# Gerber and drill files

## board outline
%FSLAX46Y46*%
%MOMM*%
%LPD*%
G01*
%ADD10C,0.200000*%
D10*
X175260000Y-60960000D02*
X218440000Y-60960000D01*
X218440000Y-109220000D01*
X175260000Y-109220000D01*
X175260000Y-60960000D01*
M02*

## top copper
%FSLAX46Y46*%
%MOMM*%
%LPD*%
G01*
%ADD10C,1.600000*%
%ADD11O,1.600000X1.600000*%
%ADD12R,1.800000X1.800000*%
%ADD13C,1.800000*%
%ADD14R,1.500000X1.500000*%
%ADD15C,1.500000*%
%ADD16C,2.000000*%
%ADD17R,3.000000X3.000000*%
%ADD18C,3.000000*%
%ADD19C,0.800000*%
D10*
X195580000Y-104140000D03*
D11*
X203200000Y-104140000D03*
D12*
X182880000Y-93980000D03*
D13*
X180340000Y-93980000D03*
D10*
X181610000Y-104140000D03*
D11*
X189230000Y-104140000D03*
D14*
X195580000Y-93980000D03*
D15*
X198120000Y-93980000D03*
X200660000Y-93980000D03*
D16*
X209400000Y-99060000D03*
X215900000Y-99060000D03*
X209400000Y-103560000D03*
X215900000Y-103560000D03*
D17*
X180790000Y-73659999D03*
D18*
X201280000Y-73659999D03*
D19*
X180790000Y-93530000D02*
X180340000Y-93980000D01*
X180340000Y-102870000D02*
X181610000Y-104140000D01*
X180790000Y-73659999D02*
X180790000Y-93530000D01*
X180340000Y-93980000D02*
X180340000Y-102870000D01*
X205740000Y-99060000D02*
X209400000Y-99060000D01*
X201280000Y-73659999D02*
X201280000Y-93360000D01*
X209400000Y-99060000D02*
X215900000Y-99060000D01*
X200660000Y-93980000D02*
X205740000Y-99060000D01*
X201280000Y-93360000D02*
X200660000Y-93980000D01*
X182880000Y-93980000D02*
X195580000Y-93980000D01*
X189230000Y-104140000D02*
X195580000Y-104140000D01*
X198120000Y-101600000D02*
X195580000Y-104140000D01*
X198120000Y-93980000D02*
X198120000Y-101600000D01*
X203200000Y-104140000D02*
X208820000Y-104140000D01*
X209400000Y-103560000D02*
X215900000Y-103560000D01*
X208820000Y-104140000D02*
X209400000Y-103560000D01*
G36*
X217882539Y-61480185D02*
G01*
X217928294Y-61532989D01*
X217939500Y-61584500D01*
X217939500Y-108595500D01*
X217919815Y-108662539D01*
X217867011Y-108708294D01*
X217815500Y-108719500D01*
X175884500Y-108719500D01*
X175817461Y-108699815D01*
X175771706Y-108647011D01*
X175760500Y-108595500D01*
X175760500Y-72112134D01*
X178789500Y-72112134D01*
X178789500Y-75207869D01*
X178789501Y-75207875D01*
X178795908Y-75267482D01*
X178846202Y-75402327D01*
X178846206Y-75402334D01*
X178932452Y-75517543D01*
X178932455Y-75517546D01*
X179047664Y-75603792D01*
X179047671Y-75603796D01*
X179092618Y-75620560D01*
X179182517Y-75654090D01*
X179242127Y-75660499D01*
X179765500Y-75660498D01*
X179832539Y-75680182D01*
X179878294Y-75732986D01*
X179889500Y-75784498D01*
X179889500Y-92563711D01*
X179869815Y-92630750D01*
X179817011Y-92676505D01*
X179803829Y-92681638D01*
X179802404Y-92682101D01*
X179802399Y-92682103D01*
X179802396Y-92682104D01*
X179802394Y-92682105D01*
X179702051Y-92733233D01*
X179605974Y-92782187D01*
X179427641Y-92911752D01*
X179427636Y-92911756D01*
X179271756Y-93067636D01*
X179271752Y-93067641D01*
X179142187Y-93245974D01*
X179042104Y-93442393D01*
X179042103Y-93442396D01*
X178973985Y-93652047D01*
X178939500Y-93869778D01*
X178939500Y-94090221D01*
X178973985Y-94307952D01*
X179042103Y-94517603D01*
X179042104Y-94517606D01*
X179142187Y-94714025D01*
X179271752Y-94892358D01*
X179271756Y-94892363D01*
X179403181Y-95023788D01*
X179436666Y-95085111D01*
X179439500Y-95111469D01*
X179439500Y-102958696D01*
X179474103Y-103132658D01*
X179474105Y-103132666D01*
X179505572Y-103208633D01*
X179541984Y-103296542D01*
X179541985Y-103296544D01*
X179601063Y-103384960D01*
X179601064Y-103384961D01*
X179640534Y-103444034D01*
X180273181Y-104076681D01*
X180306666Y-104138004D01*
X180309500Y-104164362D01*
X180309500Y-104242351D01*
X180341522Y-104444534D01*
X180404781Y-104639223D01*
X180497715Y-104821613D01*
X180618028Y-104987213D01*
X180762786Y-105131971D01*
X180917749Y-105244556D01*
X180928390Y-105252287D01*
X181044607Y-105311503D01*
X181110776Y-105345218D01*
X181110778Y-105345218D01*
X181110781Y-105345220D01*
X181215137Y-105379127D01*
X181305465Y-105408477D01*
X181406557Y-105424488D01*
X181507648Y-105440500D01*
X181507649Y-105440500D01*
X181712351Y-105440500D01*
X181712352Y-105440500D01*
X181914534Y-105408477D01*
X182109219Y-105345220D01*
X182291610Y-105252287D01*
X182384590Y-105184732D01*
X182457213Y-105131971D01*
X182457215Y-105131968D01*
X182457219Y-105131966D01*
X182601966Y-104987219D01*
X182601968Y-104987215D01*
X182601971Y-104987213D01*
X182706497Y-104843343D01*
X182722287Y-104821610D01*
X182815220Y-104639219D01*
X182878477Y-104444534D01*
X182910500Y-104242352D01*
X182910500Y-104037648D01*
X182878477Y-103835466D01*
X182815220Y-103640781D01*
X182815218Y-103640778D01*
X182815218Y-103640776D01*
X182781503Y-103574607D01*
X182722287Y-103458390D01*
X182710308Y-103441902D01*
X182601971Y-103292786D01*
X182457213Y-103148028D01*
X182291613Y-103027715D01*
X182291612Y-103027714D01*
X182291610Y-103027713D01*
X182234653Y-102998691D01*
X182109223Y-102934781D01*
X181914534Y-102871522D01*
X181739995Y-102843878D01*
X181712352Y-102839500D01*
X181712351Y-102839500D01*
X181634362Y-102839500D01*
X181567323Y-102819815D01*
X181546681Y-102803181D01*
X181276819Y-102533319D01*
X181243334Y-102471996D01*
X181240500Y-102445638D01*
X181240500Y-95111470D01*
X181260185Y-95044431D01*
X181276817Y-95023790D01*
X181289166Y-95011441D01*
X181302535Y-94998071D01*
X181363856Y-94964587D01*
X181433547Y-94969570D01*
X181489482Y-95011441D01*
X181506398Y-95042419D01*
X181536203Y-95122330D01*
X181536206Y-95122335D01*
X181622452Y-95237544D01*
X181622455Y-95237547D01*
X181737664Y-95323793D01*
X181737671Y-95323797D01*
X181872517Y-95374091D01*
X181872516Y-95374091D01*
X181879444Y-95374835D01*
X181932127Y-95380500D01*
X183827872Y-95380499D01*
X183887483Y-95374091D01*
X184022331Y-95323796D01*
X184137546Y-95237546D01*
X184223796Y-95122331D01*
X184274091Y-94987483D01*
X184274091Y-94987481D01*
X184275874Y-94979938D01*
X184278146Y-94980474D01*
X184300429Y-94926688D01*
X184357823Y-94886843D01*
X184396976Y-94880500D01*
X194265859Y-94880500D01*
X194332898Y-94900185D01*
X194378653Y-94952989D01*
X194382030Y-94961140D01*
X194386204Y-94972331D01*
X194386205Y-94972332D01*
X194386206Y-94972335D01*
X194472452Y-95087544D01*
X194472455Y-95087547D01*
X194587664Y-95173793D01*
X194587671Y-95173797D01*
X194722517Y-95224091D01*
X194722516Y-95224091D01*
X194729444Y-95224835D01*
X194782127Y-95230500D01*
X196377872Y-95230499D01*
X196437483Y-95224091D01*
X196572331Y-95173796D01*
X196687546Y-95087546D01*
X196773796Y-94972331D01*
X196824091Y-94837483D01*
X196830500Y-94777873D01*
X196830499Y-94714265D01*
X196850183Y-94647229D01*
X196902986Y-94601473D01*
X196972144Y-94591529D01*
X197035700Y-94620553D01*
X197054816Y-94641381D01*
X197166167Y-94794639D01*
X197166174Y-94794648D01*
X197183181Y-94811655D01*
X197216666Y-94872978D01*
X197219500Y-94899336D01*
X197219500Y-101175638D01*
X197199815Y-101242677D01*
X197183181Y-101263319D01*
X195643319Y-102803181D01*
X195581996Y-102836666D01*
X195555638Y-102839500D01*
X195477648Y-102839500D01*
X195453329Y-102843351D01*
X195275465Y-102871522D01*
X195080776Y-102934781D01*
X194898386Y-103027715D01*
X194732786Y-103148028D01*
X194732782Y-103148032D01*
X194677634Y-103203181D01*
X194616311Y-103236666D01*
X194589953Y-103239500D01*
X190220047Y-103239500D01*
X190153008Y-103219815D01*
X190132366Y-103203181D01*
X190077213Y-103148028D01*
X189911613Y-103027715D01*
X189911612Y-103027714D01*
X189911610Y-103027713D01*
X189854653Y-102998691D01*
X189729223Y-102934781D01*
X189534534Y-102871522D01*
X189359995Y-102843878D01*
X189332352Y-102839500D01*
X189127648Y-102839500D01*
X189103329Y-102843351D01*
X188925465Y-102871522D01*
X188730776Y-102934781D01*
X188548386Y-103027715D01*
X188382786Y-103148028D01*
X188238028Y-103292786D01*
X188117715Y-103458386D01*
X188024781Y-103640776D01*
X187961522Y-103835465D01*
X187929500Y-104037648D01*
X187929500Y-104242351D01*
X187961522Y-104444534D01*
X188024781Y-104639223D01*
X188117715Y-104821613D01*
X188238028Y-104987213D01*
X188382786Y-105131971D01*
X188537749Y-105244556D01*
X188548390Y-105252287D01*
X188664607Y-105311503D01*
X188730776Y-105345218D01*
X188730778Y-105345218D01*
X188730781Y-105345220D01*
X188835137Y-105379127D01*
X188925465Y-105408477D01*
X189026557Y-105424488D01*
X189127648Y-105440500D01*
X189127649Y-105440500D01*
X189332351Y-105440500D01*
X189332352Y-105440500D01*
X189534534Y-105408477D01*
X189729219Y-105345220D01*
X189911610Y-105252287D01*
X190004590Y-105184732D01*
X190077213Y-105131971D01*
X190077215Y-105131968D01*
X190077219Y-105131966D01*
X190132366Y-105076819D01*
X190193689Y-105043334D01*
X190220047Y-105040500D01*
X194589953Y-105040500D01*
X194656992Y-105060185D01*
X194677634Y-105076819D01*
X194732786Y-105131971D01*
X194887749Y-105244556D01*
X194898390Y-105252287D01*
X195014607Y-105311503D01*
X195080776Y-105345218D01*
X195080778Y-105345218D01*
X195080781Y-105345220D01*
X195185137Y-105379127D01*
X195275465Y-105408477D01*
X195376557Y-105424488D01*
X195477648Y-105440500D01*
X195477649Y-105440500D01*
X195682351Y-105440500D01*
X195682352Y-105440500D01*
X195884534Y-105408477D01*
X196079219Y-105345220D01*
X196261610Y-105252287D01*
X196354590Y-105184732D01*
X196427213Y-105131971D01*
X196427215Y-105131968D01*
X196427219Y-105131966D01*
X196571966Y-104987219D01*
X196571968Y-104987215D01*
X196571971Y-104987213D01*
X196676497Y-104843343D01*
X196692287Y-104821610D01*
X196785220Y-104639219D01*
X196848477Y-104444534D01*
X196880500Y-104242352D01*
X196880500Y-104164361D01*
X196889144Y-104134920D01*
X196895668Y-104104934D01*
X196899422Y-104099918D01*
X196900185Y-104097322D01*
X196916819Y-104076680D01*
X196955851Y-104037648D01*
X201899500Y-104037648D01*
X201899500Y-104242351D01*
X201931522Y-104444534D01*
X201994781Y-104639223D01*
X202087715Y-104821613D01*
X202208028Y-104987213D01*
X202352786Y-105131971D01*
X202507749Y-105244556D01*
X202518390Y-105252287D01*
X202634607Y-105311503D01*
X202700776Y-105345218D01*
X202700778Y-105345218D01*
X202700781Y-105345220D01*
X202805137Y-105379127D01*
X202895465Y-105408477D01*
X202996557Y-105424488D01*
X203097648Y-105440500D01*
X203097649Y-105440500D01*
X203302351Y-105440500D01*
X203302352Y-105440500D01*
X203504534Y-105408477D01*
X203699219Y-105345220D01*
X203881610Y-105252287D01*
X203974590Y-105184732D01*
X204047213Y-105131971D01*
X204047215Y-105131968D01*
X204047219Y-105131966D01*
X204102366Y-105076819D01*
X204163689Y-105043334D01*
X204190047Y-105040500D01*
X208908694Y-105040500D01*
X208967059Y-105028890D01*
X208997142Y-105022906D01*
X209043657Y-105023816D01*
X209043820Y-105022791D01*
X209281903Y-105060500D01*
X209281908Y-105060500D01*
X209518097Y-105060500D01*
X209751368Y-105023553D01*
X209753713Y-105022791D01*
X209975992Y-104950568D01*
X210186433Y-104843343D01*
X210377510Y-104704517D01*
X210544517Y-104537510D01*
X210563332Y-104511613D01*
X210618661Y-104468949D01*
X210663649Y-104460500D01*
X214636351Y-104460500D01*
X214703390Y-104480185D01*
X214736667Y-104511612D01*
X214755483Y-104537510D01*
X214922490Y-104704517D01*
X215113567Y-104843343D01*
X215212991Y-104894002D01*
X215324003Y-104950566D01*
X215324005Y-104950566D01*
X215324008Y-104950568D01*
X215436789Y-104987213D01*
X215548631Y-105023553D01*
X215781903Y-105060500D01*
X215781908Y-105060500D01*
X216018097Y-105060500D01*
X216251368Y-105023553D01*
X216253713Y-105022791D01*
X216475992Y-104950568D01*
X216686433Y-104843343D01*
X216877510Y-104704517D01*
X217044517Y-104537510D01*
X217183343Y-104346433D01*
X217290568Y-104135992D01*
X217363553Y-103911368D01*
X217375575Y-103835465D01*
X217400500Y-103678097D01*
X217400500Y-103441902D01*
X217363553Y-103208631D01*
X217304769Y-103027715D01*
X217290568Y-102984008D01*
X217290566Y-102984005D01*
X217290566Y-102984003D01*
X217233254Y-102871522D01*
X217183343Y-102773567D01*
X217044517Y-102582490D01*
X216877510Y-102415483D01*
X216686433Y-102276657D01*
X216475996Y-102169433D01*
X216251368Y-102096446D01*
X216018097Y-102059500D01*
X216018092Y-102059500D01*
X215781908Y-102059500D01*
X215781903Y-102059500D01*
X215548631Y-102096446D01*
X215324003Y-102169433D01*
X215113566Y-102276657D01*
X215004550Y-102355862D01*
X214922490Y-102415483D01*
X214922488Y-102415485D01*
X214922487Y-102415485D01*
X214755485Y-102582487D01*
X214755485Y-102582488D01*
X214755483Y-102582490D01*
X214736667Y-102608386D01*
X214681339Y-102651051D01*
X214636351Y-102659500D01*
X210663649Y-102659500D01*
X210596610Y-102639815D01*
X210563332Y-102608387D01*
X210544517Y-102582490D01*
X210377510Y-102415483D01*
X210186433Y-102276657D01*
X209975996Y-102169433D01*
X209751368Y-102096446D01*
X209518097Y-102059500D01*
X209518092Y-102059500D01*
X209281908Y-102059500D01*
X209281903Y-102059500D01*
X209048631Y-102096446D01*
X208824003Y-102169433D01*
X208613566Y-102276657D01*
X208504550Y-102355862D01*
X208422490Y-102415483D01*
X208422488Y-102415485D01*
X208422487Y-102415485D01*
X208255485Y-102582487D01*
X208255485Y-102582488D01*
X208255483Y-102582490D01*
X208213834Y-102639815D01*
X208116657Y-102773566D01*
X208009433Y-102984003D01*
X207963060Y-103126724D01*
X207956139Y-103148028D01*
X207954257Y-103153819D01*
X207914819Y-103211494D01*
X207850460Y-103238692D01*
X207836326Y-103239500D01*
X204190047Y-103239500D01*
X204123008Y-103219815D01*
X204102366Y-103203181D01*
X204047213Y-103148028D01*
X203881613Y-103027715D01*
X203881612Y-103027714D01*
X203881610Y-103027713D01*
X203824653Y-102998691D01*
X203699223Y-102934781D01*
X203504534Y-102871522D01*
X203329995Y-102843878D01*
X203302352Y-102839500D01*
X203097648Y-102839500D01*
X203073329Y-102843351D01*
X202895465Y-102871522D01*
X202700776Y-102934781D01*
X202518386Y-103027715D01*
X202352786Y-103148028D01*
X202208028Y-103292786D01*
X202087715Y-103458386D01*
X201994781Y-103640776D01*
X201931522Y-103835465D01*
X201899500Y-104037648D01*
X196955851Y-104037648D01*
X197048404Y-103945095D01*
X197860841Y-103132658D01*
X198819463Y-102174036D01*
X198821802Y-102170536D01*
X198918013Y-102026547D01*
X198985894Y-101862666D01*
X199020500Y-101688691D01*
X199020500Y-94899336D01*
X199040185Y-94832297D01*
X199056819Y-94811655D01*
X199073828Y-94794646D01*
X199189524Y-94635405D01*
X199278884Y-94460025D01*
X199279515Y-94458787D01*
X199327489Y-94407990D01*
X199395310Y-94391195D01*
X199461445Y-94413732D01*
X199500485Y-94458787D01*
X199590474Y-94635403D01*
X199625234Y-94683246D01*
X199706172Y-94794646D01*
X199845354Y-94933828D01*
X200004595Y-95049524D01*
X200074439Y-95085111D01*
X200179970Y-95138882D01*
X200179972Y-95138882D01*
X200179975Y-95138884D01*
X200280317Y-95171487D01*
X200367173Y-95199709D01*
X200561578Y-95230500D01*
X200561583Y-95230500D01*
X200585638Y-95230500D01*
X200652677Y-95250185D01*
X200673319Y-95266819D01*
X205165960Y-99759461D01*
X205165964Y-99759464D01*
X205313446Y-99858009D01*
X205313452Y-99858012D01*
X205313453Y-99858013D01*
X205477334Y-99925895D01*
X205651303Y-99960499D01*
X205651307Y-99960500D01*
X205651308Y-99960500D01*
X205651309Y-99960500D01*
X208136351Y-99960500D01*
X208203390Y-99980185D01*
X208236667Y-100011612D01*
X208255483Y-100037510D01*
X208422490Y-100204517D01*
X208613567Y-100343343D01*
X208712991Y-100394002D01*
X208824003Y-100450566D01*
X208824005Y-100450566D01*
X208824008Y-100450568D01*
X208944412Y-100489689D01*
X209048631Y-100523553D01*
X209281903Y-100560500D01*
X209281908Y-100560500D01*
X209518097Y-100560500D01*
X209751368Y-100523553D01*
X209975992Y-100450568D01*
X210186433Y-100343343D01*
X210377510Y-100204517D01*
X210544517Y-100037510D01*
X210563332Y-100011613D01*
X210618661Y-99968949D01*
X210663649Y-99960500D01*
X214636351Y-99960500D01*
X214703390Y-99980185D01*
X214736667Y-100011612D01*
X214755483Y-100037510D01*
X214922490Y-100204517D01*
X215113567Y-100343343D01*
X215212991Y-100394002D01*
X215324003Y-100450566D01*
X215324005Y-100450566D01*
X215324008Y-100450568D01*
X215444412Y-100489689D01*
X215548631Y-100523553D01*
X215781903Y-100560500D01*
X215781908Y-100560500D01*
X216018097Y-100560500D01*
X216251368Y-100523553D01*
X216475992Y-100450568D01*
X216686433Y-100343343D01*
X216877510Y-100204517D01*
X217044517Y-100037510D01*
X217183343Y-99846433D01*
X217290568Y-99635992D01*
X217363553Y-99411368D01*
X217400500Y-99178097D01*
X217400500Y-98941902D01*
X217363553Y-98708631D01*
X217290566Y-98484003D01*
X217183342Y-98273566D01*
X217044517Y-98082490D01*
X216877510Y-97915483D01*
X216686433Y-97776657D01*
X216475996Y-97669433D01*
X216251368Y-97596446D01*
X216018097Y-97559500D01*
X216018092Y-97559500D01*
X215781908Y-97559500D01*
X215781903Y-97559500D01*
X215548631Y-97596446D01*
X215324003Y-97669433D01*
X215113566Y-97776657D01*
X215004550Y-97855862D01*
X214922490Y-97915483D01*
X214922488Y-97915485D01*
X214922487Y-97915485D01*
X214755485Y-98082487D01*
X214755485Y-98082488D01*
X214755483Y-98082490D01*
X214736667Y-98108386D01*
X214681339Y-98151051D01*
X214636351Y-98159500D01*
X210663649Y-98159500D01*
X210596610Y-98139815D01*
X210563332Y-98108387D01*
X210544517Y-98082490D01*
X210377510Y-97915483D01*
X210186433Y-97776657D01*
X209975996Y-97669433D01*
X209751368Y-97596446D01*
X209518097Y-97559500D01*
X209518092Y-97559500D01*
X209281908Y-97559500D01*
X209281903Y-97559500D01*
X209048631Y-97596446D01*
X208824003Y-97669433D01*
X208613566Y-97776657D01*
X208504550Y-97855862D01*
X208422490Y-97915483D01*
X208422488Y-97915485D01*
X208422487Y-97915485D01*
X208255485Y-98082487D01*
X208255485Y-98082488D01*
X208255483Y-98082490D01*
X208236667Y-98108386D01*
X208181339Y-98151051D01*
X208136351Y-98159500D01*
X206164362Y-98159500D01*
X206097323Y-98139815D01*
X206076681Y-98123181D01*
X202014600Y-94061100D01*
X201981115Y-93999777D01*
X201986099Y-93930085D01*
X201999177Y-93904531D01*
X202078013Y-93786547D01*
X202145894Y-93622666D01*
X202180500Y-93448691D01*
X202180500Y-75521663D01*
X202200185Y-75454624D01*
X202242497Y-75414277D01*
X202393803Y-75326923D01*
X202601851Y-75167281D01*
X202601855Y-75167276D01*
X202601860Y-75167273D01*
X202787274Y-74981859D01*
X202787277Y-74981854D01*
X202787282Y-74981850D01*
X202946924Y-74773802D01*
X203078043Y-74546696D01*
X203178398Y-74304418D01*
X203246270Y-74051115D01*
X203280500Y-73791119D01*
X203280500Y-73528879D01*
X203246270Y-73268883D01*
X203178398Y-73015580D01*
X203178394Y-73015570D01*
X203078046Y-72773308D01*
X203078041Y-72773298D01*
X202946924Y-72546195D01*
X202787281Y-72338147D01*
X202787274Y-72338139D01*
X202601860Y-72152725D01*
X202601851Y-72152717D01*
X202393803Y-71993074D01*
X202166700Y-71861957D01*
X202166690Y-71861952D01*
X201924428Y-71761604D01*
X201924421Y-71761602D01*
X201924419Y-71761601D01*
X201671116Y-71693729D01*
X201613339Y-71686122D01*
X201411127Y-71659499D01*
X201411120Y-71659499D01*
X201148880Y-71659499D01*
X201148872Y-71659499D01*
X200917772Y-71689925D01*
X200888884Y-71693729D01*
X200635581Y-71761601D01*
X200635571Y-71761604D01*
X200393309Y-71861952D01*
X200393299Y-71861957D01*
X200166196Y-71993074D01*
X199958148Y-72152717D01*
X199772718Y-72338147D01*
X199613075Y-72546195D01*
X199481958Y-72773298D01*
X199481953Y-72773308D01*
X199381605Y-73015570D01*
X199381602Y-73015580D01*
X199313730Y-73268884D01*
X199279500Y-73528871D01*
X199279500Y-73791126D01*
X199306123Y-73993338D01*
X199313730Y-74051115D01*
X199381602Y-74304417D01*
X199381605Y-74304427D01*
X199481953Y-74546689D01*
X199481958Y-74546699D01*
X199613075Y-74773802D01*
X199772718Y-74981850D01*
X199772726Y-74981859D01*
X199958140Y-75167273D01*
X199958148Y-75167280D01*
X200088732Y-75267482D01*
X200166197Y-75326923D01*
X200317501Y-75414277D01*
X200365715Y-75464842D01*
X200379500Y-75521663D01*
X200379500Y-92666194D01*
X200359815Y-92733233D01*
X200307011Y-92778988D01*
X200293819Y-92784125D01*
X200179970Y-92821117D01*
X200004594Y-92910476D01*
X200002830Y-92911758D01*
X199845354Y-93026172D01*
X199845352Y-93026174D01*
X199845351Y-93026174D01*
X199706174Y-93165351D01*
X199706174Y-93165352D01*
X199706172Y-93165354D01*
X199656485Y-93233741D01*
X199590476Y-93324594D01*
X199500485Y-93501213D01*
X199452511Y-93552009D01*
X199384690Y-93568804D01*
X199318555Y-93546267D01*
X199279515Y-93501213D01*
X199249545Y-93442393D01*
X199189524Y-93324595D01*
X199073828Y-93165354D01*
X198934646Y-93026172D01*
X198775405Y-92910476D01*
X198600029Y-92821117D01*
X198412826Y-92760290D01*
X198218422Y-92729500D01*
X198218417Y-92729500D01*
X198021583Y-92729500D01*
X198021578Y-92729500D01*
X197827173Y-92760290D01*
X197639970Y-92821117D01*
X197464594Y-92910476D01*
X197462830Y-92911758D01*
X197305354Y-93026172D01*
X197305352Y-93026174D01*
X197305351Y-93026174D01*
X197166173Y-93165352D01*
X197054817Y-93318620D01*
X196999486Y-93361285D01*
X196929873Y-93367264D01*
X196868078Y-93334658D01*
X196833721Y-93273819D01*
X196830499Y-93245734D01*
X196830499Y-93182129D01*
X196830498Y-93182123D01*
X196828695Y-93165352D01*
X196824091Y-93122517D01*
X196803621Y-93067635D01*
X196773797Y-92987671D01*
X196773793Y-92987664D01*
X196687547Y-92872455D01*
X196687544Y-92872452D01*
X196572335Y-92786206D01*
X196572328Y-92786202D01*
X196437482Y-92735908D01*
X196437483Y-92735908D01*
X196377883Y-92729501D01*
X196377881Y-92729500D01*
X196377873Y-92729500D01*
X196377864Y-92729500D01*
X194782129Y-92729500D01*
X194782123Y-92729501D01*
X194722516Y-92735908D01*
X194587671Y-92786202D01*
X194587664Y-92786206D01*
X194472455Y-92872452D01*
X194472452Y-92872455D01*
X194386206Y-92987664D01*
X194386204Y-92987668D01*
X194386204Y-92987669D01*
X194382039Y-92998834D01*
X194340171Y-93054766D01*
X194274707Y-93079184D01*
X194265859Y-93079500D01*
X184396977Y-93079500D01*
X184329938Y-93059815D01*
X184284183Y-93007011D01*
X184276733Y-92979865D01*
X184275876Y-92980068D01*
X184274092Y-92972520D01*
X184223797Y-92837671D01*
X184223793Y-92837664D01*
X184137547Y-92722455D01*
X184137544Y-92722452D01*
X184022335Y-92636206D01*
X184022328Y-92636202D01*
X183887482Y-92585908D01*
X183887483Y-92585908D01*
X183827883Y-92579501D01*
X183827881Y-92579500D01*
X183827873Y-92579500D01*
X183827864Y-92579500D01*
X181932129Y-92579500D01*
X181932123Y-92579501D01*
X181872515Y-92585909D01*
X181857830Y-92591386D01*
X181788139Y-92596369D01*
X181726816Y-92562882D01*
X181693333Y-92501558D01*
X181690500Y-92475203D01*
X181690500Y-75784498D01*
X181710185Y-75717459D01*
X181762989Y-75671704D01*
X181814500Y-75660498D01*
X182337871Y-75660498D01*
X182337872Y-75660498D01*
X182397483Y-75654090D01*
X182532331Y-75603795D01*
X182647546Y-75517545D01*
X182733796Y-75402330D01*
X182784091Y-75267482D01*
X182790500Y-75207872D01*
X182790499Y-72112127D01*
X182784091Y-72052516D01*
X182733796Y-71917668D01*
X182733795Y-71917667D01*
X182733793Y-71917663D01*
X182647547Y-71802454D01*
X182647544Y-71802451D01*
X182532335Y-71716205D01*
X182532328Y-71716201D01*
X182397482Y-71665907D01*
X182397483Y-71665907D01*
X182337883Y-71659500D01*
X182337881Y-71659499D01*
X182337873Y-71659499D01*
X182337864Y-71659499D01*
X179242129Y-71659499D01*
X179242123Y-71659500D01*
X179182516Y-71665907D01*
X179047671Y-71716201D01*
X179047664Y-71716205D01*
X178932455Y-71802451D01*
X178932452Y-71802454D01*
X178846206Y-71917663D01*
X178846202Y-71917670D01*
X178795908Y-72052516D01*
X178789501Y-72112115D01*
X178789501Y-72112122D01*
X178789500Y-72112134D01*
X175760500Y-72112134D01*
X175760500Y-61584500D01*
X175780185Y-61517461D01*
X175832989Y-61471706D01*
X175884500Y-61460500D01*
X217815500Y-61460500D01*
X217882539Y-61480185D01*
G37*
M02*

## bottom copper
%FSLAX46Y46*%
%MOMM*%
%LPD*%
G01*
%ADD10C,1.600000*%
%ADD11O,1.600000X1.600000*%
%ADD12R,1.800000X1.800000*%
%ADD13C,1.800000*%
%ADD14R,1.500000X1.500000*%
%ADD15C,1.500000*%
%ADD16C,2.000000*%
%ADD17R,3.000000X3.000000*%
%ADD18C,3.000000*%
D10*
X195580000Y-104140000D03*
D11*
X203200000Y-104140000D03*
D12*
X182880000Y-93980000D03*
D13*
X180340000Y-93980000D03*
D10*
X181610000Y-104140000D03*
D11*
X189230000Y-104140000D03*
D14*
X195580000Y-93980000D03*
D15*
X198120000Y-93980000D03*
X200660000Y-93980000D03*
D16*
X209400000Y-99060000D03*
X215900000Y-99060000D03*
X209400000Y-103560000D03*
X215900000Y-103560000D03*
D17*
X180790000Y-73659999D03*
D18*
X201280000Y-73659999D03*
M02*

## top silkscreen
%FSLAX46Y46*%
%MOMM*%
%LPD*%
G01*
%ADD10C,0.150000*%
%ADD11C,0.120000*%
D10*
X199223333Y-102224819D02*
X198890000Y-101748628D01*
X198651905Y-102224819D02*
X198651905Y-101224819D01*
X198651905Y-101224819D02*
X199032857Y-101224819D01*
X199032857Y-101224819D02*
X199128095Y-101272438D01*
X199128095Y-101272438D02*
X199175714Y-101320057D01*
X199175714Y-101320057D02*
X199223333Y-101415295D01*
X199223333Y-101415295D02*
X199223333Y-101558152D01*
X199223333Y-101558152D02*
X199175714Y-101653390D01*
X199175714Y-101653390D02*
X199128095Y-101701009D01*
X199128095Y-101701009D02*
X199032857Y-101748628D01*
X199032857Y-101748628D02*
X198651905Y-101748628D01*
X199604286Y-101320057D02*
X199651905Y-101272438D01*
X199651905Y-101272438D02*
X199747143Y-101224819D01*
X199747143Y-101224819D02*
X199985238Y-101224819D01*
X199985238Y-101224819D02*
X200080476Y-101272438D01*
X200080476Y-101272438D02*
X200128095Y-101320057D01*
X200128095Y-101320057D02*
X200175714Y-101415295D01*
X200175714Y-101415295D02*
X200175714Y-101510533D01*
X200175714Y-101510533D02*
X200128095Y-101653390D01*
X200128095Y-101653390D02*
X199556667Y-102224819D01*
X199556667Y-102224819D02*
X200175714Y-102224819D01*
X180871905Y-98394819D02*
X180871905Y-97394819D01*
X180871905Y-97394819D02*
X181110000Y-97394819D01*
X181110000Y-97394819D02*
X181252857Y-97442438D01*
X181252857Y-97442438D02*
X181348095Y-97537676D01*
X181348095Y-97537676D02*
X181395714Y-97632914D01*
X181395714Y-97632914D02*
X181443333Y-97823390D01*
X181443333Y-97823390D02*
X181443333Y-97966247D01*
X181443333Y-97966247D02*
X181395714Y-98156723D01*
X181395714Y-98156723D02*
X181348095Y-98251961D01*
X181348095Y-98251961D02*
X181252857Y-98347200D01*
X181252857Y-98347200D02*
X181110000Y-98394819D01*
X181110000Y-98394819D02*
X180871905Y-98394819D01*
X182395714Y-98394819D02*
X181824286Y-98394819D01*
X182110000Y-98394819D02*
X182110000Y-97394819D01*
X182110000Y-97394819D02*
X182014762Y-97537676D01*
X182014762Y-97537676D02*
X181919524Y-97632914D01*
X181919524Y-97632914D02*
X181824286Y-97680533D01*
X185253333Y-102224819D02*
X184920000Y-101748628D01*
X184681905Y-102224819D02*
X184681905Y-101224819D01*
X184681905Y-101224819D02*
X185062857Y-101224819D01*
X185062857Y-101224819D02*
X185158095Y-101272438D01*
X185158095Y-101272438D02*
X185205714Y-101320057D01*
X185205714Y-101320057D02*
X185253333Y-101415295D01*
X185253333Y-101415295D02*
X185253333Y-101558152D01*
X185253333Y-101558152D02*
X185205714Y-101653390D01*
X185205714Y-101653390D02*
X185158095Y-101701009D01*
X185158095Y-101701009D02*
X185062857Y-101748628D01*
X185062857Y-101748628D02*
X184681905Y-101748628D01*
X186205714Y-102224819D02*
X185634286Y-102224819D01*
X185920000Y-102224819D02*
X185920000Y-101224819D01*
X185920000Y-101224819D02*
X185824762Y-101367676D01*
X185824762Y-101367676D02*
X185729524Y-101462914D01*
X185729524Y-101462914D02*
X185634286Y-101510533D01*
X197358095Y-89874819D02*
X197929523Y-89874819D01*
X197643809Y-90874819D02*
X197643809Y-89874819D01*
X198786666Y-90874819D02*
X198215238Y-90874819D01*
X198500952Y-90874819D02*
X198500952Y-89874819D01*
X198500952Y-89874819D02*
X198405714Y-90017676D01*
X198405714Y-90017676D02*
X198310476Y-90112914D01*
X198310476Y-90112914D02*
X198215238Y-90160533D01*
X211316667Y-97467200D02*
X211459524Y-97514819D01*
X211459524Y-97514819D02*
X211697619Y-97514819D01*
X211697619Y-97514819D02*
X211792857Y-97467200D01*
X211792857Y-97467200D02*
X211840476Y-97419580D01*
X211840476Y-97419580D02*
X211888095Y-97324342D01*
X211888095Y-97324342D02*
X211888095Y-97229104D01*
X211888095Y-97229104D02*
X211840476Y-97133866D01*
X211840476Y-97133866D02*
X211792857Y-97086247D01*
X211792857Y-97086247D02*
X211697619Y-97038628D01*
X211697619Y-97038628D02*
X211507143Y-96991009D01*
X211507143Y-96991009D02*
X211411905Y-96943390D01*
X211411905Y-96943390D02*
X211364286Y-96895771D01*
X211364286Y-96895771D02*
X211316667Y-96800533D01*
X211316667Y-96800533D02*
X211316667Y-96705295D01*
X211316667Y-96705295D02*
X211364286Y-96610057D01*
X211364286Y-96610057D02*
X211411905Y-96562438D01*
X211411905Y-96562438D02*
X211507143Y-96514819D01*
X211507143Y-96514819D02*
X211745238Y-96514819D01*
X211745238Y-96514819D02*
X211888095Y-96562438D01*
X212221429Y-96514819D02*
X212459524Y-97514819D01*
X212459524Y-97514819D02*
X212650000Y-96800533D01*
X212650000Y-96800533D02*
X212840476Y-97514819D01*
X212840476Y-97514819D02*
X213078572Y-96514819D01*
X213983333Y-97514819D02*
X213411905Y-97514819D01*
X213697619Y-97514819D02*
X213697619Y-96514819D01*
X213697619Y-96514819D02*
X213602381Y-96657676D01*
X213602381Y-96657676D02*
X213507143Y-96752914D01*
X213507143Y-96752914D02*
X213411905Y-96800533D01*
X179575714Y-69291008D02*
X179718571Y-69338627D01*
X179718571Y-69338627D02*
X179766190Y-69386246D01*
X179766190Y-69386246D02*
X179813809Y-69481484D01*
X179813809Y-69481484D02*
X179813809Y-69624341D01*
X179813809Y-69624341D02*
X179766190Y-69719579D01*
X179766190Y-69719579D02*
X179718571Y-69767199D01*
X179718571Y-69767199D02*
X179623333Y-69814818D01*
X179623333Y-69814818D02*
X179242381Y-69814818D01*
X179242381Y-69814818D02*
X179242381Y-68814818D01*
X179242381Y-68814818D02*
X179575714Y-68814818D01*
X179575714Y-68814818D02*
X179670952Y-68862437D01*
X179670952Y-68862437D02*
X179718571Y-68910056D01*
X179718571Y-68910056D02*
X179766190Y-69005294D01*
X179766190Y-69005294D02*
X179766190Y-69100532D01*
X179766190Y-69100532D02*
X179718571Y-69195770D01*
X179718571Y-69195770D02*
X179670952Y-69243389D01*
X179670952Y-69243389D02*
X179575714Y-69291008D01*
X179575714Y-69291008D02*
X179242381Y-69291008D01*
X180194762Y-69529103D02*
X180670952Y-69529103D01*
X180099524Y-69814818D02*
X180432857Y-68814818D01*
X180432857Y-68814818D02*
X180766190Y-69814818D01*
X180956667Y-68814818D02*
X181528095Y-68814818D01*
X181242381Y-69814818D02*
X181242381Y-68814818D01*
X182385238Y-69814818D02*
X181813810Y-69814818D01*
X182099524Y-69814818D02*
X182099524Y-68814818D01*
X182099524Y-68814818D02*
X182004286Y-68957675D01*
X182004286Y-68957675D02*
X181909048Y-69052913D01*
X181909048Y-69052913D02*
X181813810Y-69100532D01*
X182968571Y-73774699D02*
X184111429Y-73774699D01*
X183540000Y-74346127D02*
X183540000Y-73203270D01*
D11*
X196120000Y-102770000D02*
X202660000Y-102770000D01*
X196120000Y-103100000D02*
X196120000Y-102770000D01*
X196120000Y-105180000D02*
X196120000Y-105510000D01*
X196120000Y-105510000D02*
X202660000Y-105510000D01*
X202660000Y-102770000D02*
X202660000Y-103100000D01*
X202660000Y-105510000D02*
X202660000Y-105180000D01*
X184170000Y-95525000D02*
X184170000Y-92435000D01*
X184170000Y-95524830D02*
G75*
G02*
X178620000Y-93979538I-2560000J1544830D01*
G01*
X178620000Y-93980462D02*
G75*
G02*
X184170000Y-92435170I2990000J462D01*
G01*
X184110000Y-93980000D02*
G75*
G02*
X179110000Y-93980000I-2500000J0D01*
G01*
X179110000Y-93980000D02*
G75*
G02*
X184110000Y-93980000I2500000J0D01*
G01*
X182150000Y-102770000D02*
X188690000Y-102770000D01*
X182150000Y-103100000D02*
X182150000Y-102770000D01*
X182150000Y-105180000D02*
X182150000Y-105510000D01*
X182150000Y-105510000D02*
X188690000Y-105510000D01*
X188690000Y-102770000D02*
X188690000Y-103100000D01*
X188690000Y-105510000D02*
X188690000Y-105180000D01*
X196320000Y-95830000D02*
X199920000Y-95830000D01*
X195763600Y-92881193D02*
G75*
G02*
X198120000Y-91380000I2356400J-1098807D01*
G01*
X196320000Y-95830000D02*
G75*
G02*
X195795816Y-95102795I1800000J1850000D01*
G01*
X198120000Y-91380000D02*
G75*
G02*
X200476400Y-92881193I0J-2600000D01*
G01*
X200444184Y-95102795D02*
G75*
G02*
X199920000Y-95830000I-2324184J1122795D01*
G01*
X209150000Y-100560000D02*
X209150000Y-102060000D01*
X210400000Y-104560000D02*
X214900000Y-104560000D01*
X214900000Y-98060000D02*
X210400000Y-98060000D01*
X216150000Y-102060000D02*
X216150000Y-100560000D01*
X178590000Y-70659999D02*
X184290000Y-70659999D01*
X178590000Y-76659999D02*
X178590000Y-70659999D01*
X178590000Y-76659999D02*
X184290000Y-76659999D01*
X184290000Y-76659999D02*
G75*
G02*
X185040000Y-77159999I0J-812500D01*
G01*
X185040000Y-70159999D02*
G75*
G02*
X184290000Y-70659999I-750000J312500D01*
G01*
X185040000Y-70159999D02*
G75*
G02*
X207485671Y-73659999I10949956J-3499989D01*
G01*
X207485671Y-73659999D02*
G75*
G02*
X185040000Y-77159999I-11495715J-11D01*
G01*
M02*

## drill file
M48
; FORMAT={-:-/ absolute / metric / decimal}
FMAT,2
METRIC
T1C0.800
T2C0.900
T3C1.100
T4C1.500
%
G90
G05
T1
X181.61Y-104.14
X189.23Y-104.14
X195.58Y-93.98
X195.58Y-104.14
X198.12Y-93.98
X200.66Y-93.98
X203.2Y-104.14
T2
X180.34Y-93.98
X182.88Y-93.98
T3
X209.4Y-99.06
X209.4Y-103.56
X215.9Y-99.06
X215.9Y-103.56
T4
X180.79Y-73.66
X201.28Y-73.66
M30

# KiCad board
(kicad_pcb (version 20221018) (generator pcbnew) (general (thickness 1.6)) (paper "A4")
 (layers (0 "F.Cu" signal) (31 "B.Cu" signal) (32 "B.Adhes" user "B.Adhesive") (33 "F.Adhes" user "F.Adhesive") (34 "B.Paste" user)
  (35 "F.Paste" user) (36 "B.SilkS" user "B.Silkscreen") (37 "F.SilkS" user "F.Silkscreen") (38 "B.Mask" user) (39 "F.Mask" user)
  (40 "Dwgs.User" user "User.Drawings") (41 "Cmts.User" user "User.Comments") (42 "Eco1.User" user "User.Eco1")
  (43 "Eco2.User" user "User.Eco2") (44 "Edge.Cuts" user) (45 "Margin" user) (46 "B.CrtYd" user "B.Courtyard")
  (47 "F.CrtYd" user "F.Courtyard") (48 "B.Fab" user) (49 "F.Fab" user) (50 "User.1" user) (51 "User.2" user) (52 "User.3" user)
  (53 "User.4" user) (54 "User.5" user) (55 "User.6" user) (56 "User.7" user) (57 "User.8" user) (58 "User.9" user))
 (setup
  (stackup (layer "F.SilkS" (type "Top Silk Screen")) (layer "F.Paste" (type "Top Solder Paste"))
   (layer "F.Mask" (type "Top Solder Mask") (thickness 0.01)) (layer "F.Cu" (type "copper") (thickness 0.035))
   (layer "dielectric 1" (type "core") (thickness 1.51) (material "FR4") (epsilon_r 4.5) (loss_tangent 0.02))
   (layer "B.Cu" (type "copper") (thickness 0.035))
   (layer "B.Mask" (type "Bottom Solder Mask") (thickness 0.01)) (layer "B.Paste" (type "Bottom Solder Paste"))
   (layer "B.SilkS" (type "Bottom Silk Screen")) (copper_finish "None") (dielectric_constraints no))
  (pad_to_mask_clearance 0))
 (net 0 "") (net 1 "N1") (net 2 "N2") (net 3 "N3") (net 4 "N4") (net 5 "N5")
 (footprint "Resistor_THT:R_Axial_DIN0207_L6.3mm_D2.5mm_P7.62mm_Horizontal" (layer "F.Cu") (at 195.58 104.14)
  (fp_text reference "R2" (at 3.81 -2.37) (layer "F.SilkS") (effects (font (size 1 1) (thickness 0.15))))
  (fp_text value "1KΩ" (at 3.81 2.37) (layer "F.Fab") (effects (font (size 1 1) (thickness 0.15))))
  (fp_line (start 0.54 -1.37) (end 7.08 -1.37) (stroke (width 0.12) (type solid)) (layer "F.SilkS"))
  (fp_line (start 0.54 -1.04) (end 0.54 -1.37) (stroke (width 0.12) (type solid)) (layer "F.SilkS"))
  (fp_line (start 0.54 1.04) (end 0.54 1.37) (stroke (width 0.12) (type solid)) (layer "F.SilkS"))
  (fp_line (start 0.54 1.37) (end 7.08 1.37) (stroke (width 0.12) (type solid)) (layer "F.SilkS"))
  (fp_line (start 7.08 -1.37) (end 7.08 -1.04) (stroke (width 0.12) (type solid)) (layer "F.SilkS"))
  (fp_line (start 7.08 1.37) (end 7.08 1.04) (stroke (width 0.12) (type solid)) (layer "F.SilkS"))
  (pad "1" thru_hole circle (at 0 0) (size 1.6 1.6) (drill 0.8) (layers "*.Cu" "*.Mask") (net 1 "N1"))
  (pad "2" thru_hole oval (at 7.62 0) (size 1.6 1.6) (drill 0.8) (layers "*.Cu" "*.Mask") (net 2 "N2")))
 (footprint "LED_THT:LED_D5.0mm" (layer "F.Cu") (at 182.88 93.98 180)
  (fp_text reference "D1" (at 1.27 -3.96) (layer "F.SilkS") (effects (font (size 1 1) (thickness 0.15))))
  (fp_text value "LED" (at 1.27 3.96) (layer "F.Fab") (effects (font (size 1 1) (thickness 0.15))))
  (fp_line (start -1.29 -1.545) (end -1.29 1.545) (stroke (width 0.12) (type solid)) (layer "F.SilkS"))
  (fp_arc (start -1.29 -1.54483) (mid 2.072002 -2.880433) (end 4.26 0.000462) (stroke (width 0.12) (type solid)) (layer "F.SilkS"))
  (fp_arc (start 4.26 -0.000462) (mid 2.072002 2.880433) (end -1.29 1.54483) (stroke (width 0.12) (type solid)) (layer "F.SilkS"))
  (fp_circle (center 1.27 0) (end 3.77 0) (stroke (width 0.12) (type solid)) (fill none) (layer "F.SilkS"))
  (pad "1" thru_hole rect (at 0 0 180) (size 1.8 1.8) (drill 0.9) (layers "*.Cu" "*.Mask") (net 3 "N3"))
  (pad "2" thru_hole circle (at 2.54 0 180) (size 1.8 1.8) (drill 0.9) (layers "*.Cu" "*.Mask") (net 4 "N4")))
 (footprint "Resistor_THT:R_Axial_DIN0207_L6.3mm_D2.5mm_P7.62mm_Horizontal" (layer "F.Cu") (at 181.61 104.14)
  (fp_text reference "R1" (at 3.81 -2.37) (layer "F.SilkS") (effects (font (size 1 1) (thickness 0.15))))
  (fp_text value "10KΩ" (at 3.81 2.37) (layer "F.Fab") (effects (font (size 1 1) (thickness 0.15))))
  (fp_line (start 0.54 -1.37) (end 7.08 -1.37) (stroke (width 0.12) (type solid)) (layer "F.SilkS"))
  (fp_line (start 0.54 -1.04) (end 0.54 -1.37) (stroke (width 0.12) (type solid)) (layer "F.SilkS"))
  (fp_line (start 0.54 1.04) (end 0.54 1.37) (stroke (width 0.12) (type solid)) (layer "F.SilkS"))
  (fp_line (start 0.54 1.37) (end 7.08 1.37) (stroke (width 0.12) (type solid)) (layer "F.SilkS"))
  (fp_line (start 7.08 -1.37) (end 7.08 -1.04) (stroke (width 0.12) (type solid)) (layer "F.SilkS"))
  (fp_line (start 7.08 1.37) (end 7.08 1.04) (stroke (width 0.12) (type solid)) (layer "F.SilkS"))
  (pad "1" thru_hole circle (at 0 0) (size 1.6 1.6) (drill 0.8) (layers "*.Cu" "*.Mask") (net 4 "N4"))
  (pad "2" thru_hole oval (at 7.62 0) (size 1.6 1.6) (drill 0.8) (layers "*.Cu" "*.Mask") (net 1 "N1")))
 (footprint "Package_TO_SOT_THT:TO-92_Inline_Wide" (layer "F.Cu") (at 195.58 93.98)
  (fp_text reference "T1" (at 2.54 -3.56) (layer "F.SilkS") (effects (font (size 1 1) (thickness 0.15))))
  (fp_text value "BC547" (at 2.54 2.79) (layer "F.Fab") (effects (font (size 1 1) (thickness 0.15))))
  (fp_line (start 0.74 1.85) (end 4.34 1.85) (stroke (width 0.12) (type solid)) (layer "F.SilkS"))
  (fp_arc (start 0.1836 -1.098807) (mid 1.143021 -2.192817) (end 2.54 -2.6) (stroke (width 0.12) (type solid)) (layer "F.SilkS"))
  (fp_arc (start 0.74 1.85) (mid 0.446097 1.509328) (end 0.215816 1.122795) (stroke (width 0.12) (type solid)) (layer "F.SilkS"))
  (fp_arc (start 2.54 -2.6) (mid 3.936979 -2.192818) (end 4.8964 -1.098807) (stroke (width 0.12) (type solid)) (layer "F.SilkS"))
  (fp_arc (start 4.864184 1.122795) (mid 4.633903 1.509328) (end 4.34 1.85) (stroke (width 0.12) (type solid)) (layer "F.SilkS"))
  (pad "1" thru_hole rect (at 0 0) (size 1.5 1.5) (drill 0.8) (layers "*.Cu" "*.Mask") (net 3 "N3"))
  (pad "2" thru_hole circle (at 2.54 0) (size 1.5 1.5) (drill 0.8) (layers "*.Cu" "*.Mask") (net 1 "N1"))
  (pad "3" thru_hole circle (at 5.08 0) (size 1.5 1.5) (drill 0.8) (layers "*.Cu" "*.Mask") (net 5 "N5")))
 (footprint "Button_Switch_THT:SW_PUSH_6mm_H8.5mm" (layer "F.Cu") (at 209.4 99.06)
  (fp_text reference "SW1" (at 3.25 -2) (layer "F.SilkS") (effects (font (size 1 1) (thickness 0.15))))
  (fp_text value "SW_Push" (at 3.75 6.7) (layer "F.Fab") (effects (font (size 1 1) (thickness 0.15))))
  (fp_line (start -0.25 1.5) (end -0.25 3) (stroke (width 0.12) (type solid)) (layer "F.SilkS"))
  (fp_line (start 1 5.5) (end 5.5 5.5) (stroke (width 0.12) (type solid)) (layer "F.SilkS"))
  (fp_line (start 5.5 -1) (end 1 -1) (stroke (width 0.12) (type solid)) (layer "F.SilkS"))
  (fp_line (start 6.75 3) (end 6.75 1.5) (stroke (width 0.12) (type solid)) (layer "F.SilkS"))
  (pad "1" thru_hole circle (at 0 0 90) (size 2 2) (drill 1.1) (layers "*.Cu" "*.Mask") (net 5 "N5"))
  (pad "1" thru_hole circle (at 6.5 0 90) (size 2 2) (drill 1.1) (layers "*.Cu" "*.Mask") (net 5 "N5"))
  (pad "2" thru_hole circle (at 0 4.5 90) (size 2 2) (drill 1.1) (layers "*.Cu" "*.Mask") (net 2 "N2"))
  (pad "2" thru_hole circle (at 6.5 4.5 90) (size 2 2) (drill 1.1) (layers "*.Cu" "*.Mask") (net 2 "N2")))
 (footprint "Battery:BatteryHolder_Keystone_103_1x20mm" (layer "F.Cu") (at 180.79 73.659999)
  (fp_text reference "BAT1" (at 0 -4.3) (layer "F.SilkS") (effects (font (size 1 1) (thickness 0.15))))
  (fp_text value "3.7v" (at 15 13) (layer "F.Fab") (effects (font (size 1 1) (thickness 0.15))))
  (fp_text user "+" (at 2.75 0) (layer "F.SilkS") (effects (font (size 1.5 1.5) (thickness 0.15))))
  (fp_line (start -2.2 -3) (end 3.5 -3) (stroke (width 0.12) (type solid)) (layer "F.SilkS"))
  (fp_line (start -2.2 3) (end -2.2 -3) (stroke (width 0.12) (type solid)) (layer "F.SilkS"))
  (fp_line (start -2.2 3) (end 3.5 3) (stroke (width 0.12) (type solid)) (layer "F.SilkS"))
  (fp_arc (start 3.5 3) (mid 3.950694 3.136459) (end 4.25 3.5) (stroke (width 0.12) (type solid)) (layer "F.SilkS"))
  (fp_arc (start 4.25 -3.5) (mid 3.950694 -3.136459) (end 3.5 -3) (stroke (width 0.12) (type solid)) (layer "F.SilkS"))
  (fp_arc (start 4.25 -3.5) (mid 16.971103 -11.358466) (end 26.695671 0) (stroke (width 0.12) (type solid)) (layer "F.SilkS"))
  (fp_arc (start 26.695671 0) (mid 16.971103 11.358466) (end 4.25 3.5) (stroke (width 0.12) (type solid)) (layer "F.SilkS"))
  (pad "1" thru_hole rect (at 0 0) (size 3 3) (drill 1.5) (layers "*.Cu" "*.Mask") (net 4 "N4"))
  (pad "2" thru_hole circle (at 20.49 0) (size 3 3) (drill 1.5) (layers "*.Cu" "*.Mask") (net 5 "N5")))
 (gr_rect (start 175.26 60.96) (end 218.44 109.22) (stroke (width 0.2) (type default)) (fill none) (layer "Edge.Cuts"))
 (segment (start 180.79 93.53) (end 180.34 93.98) (width 0.8) (layer "F.Cu") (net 4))
 (segment (start 180.34 102.87) (end 181.61 104.14) (width 0.8) (layer "F.Cu") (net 4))
 (segment (start 180.79 73.659999) (end 180.79 93.53) (width 0.8) (layer "F.Cu") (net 4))
 (segment (start 180.34 93.98) (end 180.34 102.87) (width 0.8) (layer "F.Cu") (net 4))
 (segment (start 205.74 99.06) (end 209.4 99.06) (width 0.8) (layer "F.Cu") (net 5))
 (segment (start 201.28 73.659999) (end 201.28 93.36) (width 0.8) (layer "F.Cu") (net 5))
 (segment (start 209.4 99.06) (end 215.9 99.06) (width 0.8) (layer "F.Cu") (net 5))
 (segment (start 200.66 93.98) (end 205.74 99.06) (width 0.8) (layer "F.Cu") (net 5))
 (segment (start 201.28 93.36) (end 200.66 93.98) (width 0.8) (layer "F.Cu") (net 5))
 (segment (start 182.88 93.98) (end 195.58 93.98) (width 0.8) (layer "F.Cu") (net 3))
 (segment (start 189.23 104.14) (end 195.58 104.14) (width 0.8) (layer "F.Cu") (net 1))
 (segment (start 198.12 101.6) (end 195.58 104.14) (width 0.8) (layer "F.Cu") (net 1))
 (segment (start 198.12 93.98) (end 198.12 101.6) (width 0.8) (layer "F.Cu") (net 1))
 (segment (start 203.2 104.14) (end 208.82 104.14) (width 0.8) (layer "F.Cu") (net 2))
 (segment (start 209.4 103.56) (end 215.9 103.56) (width 0.8) (layer "F.Cu") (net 2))
 (segment (start 208.82 104.14) (end 209.4 103.56) (width 0.8) (layer "F.Cu") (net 2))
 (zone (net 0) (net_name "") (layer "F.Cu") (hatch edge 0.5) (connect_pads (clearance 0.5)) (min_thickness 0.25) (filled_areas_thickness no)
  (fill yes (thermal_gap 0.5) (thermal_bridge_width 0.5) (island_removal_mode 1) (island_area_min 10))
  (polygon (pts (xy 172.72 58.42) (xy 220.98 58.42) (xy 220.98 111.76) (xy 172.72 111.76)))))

